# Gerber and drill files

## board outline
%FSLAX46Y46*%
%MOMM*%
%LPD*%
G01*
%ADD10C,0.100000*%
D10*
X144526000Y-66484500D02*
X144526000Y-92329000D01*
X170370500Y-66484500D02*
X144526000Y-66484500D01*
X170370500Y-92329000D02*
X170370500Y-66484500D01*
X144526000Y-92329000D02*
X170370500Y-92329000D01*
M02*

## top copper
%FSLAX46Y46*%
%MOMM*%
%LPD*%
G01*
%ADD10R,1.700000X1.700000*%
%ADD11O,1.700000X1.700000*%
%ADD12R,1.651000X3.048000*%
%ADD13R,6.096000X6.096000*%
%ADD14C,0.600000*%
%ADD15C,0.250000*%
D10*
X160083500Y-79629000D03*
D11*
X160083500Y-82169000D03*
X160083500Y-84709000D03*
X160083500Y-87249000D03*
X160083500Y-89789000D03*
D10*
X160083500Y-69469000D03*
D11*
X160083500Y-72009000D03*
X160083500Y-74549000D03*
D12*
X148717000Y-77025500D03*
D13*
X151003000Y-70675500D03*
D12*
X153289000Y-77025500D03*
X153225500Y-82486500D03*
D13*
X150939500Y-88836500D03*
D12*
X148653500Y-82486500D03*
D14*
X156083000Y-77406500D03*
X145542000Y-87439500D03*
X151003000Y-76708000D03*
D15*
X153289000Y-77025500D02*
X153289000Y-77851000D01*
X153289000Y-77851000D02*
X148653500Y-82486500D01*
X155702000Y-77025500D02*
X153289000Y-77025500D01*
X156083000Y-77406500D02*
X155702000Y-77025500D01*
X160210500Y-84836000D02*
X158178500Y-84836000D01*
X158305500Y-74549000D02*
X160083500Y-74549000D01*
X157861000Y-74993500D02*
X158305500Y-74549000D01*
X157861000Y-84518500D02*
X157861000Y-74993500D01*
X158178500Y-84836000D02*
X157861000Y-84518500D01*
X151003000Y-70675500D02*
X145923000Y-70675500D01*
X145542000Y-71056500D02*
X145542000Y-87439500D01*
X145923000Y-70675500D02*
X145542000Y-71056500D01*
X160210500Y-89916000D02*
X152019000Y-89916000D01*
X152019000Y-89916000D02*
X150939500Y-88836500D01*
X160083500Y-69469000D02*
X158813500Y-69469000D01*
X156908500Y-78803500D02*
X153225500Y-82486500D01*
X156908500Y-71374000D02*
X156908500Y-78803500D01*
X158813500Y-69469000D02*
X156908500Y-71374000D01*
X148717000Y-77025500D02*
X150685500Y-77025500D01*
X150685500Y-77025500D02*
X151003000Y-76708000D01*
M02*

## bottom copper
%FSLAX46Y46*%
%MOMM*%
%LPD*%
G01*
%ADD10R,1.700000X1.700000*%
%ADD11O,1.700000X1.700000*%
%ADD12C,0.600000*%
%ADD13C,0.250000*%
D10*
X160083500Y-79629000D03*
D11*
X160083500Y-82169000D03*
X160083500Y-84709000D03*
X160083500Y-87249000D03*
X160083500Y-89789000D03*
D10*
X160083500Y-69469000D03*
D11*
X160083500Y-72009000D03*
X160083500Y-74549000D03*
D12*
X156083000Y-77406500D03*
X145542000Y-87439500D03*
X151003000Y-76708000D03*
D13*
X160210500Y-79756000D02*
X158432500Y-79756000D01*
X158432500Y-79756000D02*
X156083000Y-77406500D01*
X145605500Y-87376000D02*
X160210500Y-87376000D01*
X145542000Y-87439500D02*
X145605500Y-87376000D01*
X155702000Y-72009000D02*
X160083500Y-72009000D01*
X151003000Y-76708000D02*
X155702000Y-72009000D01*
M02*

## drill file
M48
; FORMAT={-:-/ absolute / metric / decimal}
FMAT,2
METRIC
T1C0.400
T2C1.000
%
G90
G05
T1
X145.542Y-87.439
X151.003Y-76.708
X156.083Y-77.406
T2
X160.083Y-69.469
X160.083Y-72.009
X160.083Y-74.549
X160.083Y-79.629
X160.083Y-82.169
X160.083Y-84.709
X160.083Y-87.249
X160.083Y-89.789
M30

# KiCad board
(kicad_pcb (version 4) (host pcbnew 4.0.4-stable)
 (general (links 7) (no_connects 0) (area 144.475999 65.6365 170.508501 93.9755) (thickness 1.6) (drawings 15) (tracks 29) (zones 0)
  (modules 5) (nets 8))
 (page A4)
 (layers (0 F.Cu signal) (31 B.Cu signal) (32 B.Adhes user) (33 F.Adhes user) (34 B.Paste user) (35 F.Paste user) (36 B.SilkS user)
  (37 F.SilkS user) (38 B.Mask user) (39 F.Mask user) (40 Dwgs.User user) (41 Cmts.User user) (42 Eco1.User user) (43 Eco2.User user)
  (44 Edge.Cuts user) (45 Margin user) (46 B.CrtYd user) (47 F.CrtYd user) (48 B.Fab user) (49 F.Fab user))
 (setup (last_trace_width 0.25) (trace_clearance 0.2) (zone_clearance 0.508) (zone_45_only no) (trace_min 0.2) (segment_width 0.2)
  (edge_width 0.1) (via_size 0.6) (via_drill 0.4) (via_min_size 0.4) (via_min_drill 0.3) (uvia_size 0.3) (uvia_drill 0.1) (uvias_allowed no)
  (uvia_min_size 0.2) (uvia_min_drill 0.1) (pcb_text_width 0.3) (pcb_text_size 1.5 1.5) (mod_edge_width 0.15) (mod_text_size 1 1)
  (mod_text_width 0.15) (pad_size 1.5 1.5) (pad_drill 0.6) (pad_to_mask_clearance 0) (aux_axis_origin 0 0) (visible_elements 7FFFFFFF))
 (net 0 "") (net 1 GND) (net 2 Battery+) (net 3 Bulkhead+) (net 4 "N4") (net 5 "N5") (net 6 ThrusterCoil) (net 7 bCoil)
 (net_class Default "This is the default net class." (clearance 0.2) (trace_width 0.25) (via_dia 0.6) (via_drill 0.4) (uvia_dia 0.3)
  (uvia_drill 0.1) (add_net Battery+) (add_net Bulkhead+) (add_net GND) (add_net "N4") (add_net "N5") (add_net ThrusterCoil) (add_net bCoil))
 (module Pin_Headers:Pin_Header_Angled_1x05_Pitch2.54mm (layer F.Cu) (at 160.0835 79.629)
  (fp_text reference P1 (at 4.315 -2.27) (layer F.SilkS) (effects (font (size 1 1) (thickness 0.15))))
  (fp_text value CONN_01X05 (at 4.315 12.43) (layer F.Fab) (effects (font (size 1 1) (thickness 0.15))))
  (pad 1 thru_hole rect (at 0 0) (size 1.7 1.7) (drill 1) (layers *.Cu *.Mask) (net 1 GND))
  (pad 2 thru_hole oval (at 0 2.54) (size 1.7 1.7) (drill 1) (layers *.Cu *.Mask) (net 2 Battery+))
  (pad 3 thru_hole oval (at 0 5.08) (size 1.7 1.7) (drill 1) (layers *.Cu *.Mask) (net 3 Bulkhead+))
  (pad 4 thru_hole oval (at 0 7.62) (size 1.7 1.7) (drill 1) (layers *.Cu *.Mask) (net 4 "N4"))
  (pad 5 thru_hole oval (at 0 10.16) (size 1.7 1.7) (drill 1) (layers *.Cu *.Mask) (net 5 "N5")))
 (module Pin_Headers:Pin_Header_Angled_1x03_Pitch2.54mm (layer F.Cu) (at 160.0835 69.469)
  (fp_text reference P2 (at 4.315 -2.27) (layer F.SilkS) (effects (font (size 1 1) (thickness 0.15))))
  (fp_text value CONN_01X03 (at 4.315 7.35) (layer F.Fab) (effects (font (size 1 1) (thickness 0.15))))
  (pad 1 thru_hole rect (at 0 0) (size 1.7 1.7) (drill 1) (layers *.Cu *.Mask) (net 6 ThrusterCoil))
  (pad 2 thru_hole oval (at 0 2.54) (size 1.7 1.7) (drill 1) (layers *.Cu *.Mask) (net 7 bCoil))
  (pad 3 thru_hole oval (at 0 5.08) (size 1.7 1.7) (drill 1) (layers *.Cu *.Mask) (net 3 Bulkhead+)))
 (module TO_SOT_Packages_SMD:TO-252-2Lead (layer F.Cu) (at 151.003 77.0255)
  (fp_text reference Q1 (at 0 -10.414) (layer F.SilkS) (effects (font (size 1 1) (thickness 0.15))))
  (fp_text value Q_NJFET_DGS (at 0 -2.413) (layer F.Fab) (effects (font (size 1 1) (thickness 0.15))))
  (pad 1 smd rect (at -2.286 0) (size 1.651 3.048) (layers F.Cu F.Paste F.Mask) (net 7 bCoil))
  (pad 2 smd rect (at 0 -6.35) (size 6.096 6.096) (layers F.Cu F.Paste F.Mask) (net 4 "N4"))
  (pad 3 smd rect (at 2.286 0) (size 1.651 3.048) (layers F.Cu F.Paste F.Mask) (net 1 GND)))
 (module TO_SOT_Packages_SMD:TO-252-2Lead (layer F.Cu) (at 150.9395 82.4865 180)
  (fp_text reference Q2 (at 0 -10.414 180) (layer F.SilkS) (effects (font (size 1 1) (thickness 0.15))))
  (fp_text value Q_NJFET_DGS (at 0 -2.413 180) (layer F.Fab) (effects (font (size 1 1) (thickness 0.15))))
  (pad 1 smd rect (at -2.286 0 180) (size 1.651 3.048) (layers F.Cu F.Paste F.Mask) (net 6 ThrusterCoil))
  (pad 2 smd rect (at 0 -6.35 180) (size 6.096 6.096) (layers F.Cu F.Paste F.Mask) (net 5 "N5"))
  (pad 3 smd rect (at 2.286 0 180) (size 1.651 3.048) (layers F.Cu F.Paste F.Mask) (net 1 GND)))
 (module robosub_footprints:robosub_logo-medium (layer B.Cu) (at 151.9555 71.1835 180)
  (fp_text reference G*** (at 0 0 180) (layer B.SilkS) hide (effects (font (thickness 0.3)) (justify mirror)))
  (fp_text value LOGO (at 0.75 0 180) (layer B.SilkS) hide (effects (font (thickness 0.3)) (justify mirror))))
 (gr_line (start 144.526 66.4845) (end 144.526 92.329) (angle 90) (layer Edge.Cuts) (width 0.1))
 (gr_line (start 170.3705 66.4845) (end 144.526 66.4845) (angle 90) (layer Edge.Cuts) (width 0.1))
 (gr_line (start 170.3705 92.329) (end 170.3705 66.4845) (angle 90) (layer Edge.Cuts) (width 0.1))
 (gr_line (start 144.526 92.329) (end 170.3705 92.329) (angle 90) (layer Edge.Cuts) (width 0.1))
 (segment (start 153.289 77.0255) (end 153.289 77.851) (width 0.25) (layer F.Cu) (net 1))
 (segment (start 153.289 77.851) (end 148.6535 82.4865) (width 0.25) (layer F.Cu) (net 1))
 (segment (start 160.2105 79.756) (end 158.4325 79.756) (width 0.25) (layer B.Cu) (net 1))
 (segment (start 155.702 77.0255) (end 153.289 77.0255) (width 0.25) (layer F.Cu) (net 1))
 (segment (start 156.083 77.4065) (end 155.702 77.0255) (width 0.25) (layer F.Cu) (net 1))
 (via (at 156.083 77.4065) (size 0.6) (drill 0.4) (layers F.Cu B.Cu) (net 1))
 (segment (start 158.4325 79.756) (end 156.083 77.4065) (width 0.25) (layer B.Cu) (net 1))
 (segment (start 160.2105 84.836) (end 158.1785 84.836) (width 0.25) (layer F.Cu) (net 3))
 (segment (start 158.3055 74.549) (end 160.0835 74.549) (width 0.25) (layer F.Cu) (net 3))
 (segment (start 157.861 74.9935) (end 158.3055 74.549) (width 0.25) (layer F.Cu) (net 3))
 (segment (start 157.861 84.5185) (end 157.861 74.9935) (width 0.25) (layer F.Cu) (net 3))
 (segment (start 158.1785 84.836) (end 157.861 84.5185) (width 0.25) (layer F.Cu) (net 3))
 (segment (start 151.003 70.6755) (end 145.923 70.6755) (width 0.25) (layer F.Cu) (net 4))
 (segment (start 145.6055 87.376) (end 160.2105 87.376) (width 0.25) (layer B.Cu) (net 4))
 (segment (start 145.542 87.4395) (end 145.6055 87.376) (width 0.25) (layer B.Cu) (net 4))
 (via (at 145.542 87.4395) (size 0.6) (drill 0.4) (layers F.Cu B.Cu) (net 4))
 (segment (start 145.542 71.0565) (end 145.542 87.4395) (width 0.25) (layer F.Cu) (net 4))
 (segment (start 145.923 70.6755) (end 145.542 71.0565) (width 0.25) (layer F.Cu) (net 4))
 (segment (start 160.2105 89.916) (end 152.019 89.916) (width 0.25) (layer F.Cu) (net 5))
 (segment (start 152.019 89.916) (end 150.9395 88.8365) (width 0.25) (layer F.Cu) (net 5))
 (segment (start 160.0835 69.469) (end 158.8135 69.469) (width 0.25) (layer F.Cu) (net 6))
 (segment (start 156.9085 78.8035) (end 153.2255 82.4865) (width 0.25) (layer F.Cu) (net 6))
 (segment (start 156.9085 71.374) (end 156.9085 78.8035) (width 0.25) (layer F.Cu) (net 6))
 (segment (start 158.8135 69.469) (end 156.9085 71.374) (width 0.25) (layer F.Cu) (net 6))
 (segment (start 148.717 77.0255) (end 150.6855 77.0255) (width 0.25) (layer F.Cu) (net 7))
 (segment (start 155.702 72.009) (end 160.0835 72.009) (width 0.25) (layer B.Cu) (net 7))
 (segment (start 151.003 76.708) (end 155.702 72.009) (width 0.25) (layer B.Cu) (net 7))
 (via (at 151.003 76.708) (size 0.6) (drill 0.4) (layers F.Cu B.Cu) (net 7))
 (segment (start 150.6855 77.0255) (end 151.003 76.708) (width 0.25) (layer F.Cu) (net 7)))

